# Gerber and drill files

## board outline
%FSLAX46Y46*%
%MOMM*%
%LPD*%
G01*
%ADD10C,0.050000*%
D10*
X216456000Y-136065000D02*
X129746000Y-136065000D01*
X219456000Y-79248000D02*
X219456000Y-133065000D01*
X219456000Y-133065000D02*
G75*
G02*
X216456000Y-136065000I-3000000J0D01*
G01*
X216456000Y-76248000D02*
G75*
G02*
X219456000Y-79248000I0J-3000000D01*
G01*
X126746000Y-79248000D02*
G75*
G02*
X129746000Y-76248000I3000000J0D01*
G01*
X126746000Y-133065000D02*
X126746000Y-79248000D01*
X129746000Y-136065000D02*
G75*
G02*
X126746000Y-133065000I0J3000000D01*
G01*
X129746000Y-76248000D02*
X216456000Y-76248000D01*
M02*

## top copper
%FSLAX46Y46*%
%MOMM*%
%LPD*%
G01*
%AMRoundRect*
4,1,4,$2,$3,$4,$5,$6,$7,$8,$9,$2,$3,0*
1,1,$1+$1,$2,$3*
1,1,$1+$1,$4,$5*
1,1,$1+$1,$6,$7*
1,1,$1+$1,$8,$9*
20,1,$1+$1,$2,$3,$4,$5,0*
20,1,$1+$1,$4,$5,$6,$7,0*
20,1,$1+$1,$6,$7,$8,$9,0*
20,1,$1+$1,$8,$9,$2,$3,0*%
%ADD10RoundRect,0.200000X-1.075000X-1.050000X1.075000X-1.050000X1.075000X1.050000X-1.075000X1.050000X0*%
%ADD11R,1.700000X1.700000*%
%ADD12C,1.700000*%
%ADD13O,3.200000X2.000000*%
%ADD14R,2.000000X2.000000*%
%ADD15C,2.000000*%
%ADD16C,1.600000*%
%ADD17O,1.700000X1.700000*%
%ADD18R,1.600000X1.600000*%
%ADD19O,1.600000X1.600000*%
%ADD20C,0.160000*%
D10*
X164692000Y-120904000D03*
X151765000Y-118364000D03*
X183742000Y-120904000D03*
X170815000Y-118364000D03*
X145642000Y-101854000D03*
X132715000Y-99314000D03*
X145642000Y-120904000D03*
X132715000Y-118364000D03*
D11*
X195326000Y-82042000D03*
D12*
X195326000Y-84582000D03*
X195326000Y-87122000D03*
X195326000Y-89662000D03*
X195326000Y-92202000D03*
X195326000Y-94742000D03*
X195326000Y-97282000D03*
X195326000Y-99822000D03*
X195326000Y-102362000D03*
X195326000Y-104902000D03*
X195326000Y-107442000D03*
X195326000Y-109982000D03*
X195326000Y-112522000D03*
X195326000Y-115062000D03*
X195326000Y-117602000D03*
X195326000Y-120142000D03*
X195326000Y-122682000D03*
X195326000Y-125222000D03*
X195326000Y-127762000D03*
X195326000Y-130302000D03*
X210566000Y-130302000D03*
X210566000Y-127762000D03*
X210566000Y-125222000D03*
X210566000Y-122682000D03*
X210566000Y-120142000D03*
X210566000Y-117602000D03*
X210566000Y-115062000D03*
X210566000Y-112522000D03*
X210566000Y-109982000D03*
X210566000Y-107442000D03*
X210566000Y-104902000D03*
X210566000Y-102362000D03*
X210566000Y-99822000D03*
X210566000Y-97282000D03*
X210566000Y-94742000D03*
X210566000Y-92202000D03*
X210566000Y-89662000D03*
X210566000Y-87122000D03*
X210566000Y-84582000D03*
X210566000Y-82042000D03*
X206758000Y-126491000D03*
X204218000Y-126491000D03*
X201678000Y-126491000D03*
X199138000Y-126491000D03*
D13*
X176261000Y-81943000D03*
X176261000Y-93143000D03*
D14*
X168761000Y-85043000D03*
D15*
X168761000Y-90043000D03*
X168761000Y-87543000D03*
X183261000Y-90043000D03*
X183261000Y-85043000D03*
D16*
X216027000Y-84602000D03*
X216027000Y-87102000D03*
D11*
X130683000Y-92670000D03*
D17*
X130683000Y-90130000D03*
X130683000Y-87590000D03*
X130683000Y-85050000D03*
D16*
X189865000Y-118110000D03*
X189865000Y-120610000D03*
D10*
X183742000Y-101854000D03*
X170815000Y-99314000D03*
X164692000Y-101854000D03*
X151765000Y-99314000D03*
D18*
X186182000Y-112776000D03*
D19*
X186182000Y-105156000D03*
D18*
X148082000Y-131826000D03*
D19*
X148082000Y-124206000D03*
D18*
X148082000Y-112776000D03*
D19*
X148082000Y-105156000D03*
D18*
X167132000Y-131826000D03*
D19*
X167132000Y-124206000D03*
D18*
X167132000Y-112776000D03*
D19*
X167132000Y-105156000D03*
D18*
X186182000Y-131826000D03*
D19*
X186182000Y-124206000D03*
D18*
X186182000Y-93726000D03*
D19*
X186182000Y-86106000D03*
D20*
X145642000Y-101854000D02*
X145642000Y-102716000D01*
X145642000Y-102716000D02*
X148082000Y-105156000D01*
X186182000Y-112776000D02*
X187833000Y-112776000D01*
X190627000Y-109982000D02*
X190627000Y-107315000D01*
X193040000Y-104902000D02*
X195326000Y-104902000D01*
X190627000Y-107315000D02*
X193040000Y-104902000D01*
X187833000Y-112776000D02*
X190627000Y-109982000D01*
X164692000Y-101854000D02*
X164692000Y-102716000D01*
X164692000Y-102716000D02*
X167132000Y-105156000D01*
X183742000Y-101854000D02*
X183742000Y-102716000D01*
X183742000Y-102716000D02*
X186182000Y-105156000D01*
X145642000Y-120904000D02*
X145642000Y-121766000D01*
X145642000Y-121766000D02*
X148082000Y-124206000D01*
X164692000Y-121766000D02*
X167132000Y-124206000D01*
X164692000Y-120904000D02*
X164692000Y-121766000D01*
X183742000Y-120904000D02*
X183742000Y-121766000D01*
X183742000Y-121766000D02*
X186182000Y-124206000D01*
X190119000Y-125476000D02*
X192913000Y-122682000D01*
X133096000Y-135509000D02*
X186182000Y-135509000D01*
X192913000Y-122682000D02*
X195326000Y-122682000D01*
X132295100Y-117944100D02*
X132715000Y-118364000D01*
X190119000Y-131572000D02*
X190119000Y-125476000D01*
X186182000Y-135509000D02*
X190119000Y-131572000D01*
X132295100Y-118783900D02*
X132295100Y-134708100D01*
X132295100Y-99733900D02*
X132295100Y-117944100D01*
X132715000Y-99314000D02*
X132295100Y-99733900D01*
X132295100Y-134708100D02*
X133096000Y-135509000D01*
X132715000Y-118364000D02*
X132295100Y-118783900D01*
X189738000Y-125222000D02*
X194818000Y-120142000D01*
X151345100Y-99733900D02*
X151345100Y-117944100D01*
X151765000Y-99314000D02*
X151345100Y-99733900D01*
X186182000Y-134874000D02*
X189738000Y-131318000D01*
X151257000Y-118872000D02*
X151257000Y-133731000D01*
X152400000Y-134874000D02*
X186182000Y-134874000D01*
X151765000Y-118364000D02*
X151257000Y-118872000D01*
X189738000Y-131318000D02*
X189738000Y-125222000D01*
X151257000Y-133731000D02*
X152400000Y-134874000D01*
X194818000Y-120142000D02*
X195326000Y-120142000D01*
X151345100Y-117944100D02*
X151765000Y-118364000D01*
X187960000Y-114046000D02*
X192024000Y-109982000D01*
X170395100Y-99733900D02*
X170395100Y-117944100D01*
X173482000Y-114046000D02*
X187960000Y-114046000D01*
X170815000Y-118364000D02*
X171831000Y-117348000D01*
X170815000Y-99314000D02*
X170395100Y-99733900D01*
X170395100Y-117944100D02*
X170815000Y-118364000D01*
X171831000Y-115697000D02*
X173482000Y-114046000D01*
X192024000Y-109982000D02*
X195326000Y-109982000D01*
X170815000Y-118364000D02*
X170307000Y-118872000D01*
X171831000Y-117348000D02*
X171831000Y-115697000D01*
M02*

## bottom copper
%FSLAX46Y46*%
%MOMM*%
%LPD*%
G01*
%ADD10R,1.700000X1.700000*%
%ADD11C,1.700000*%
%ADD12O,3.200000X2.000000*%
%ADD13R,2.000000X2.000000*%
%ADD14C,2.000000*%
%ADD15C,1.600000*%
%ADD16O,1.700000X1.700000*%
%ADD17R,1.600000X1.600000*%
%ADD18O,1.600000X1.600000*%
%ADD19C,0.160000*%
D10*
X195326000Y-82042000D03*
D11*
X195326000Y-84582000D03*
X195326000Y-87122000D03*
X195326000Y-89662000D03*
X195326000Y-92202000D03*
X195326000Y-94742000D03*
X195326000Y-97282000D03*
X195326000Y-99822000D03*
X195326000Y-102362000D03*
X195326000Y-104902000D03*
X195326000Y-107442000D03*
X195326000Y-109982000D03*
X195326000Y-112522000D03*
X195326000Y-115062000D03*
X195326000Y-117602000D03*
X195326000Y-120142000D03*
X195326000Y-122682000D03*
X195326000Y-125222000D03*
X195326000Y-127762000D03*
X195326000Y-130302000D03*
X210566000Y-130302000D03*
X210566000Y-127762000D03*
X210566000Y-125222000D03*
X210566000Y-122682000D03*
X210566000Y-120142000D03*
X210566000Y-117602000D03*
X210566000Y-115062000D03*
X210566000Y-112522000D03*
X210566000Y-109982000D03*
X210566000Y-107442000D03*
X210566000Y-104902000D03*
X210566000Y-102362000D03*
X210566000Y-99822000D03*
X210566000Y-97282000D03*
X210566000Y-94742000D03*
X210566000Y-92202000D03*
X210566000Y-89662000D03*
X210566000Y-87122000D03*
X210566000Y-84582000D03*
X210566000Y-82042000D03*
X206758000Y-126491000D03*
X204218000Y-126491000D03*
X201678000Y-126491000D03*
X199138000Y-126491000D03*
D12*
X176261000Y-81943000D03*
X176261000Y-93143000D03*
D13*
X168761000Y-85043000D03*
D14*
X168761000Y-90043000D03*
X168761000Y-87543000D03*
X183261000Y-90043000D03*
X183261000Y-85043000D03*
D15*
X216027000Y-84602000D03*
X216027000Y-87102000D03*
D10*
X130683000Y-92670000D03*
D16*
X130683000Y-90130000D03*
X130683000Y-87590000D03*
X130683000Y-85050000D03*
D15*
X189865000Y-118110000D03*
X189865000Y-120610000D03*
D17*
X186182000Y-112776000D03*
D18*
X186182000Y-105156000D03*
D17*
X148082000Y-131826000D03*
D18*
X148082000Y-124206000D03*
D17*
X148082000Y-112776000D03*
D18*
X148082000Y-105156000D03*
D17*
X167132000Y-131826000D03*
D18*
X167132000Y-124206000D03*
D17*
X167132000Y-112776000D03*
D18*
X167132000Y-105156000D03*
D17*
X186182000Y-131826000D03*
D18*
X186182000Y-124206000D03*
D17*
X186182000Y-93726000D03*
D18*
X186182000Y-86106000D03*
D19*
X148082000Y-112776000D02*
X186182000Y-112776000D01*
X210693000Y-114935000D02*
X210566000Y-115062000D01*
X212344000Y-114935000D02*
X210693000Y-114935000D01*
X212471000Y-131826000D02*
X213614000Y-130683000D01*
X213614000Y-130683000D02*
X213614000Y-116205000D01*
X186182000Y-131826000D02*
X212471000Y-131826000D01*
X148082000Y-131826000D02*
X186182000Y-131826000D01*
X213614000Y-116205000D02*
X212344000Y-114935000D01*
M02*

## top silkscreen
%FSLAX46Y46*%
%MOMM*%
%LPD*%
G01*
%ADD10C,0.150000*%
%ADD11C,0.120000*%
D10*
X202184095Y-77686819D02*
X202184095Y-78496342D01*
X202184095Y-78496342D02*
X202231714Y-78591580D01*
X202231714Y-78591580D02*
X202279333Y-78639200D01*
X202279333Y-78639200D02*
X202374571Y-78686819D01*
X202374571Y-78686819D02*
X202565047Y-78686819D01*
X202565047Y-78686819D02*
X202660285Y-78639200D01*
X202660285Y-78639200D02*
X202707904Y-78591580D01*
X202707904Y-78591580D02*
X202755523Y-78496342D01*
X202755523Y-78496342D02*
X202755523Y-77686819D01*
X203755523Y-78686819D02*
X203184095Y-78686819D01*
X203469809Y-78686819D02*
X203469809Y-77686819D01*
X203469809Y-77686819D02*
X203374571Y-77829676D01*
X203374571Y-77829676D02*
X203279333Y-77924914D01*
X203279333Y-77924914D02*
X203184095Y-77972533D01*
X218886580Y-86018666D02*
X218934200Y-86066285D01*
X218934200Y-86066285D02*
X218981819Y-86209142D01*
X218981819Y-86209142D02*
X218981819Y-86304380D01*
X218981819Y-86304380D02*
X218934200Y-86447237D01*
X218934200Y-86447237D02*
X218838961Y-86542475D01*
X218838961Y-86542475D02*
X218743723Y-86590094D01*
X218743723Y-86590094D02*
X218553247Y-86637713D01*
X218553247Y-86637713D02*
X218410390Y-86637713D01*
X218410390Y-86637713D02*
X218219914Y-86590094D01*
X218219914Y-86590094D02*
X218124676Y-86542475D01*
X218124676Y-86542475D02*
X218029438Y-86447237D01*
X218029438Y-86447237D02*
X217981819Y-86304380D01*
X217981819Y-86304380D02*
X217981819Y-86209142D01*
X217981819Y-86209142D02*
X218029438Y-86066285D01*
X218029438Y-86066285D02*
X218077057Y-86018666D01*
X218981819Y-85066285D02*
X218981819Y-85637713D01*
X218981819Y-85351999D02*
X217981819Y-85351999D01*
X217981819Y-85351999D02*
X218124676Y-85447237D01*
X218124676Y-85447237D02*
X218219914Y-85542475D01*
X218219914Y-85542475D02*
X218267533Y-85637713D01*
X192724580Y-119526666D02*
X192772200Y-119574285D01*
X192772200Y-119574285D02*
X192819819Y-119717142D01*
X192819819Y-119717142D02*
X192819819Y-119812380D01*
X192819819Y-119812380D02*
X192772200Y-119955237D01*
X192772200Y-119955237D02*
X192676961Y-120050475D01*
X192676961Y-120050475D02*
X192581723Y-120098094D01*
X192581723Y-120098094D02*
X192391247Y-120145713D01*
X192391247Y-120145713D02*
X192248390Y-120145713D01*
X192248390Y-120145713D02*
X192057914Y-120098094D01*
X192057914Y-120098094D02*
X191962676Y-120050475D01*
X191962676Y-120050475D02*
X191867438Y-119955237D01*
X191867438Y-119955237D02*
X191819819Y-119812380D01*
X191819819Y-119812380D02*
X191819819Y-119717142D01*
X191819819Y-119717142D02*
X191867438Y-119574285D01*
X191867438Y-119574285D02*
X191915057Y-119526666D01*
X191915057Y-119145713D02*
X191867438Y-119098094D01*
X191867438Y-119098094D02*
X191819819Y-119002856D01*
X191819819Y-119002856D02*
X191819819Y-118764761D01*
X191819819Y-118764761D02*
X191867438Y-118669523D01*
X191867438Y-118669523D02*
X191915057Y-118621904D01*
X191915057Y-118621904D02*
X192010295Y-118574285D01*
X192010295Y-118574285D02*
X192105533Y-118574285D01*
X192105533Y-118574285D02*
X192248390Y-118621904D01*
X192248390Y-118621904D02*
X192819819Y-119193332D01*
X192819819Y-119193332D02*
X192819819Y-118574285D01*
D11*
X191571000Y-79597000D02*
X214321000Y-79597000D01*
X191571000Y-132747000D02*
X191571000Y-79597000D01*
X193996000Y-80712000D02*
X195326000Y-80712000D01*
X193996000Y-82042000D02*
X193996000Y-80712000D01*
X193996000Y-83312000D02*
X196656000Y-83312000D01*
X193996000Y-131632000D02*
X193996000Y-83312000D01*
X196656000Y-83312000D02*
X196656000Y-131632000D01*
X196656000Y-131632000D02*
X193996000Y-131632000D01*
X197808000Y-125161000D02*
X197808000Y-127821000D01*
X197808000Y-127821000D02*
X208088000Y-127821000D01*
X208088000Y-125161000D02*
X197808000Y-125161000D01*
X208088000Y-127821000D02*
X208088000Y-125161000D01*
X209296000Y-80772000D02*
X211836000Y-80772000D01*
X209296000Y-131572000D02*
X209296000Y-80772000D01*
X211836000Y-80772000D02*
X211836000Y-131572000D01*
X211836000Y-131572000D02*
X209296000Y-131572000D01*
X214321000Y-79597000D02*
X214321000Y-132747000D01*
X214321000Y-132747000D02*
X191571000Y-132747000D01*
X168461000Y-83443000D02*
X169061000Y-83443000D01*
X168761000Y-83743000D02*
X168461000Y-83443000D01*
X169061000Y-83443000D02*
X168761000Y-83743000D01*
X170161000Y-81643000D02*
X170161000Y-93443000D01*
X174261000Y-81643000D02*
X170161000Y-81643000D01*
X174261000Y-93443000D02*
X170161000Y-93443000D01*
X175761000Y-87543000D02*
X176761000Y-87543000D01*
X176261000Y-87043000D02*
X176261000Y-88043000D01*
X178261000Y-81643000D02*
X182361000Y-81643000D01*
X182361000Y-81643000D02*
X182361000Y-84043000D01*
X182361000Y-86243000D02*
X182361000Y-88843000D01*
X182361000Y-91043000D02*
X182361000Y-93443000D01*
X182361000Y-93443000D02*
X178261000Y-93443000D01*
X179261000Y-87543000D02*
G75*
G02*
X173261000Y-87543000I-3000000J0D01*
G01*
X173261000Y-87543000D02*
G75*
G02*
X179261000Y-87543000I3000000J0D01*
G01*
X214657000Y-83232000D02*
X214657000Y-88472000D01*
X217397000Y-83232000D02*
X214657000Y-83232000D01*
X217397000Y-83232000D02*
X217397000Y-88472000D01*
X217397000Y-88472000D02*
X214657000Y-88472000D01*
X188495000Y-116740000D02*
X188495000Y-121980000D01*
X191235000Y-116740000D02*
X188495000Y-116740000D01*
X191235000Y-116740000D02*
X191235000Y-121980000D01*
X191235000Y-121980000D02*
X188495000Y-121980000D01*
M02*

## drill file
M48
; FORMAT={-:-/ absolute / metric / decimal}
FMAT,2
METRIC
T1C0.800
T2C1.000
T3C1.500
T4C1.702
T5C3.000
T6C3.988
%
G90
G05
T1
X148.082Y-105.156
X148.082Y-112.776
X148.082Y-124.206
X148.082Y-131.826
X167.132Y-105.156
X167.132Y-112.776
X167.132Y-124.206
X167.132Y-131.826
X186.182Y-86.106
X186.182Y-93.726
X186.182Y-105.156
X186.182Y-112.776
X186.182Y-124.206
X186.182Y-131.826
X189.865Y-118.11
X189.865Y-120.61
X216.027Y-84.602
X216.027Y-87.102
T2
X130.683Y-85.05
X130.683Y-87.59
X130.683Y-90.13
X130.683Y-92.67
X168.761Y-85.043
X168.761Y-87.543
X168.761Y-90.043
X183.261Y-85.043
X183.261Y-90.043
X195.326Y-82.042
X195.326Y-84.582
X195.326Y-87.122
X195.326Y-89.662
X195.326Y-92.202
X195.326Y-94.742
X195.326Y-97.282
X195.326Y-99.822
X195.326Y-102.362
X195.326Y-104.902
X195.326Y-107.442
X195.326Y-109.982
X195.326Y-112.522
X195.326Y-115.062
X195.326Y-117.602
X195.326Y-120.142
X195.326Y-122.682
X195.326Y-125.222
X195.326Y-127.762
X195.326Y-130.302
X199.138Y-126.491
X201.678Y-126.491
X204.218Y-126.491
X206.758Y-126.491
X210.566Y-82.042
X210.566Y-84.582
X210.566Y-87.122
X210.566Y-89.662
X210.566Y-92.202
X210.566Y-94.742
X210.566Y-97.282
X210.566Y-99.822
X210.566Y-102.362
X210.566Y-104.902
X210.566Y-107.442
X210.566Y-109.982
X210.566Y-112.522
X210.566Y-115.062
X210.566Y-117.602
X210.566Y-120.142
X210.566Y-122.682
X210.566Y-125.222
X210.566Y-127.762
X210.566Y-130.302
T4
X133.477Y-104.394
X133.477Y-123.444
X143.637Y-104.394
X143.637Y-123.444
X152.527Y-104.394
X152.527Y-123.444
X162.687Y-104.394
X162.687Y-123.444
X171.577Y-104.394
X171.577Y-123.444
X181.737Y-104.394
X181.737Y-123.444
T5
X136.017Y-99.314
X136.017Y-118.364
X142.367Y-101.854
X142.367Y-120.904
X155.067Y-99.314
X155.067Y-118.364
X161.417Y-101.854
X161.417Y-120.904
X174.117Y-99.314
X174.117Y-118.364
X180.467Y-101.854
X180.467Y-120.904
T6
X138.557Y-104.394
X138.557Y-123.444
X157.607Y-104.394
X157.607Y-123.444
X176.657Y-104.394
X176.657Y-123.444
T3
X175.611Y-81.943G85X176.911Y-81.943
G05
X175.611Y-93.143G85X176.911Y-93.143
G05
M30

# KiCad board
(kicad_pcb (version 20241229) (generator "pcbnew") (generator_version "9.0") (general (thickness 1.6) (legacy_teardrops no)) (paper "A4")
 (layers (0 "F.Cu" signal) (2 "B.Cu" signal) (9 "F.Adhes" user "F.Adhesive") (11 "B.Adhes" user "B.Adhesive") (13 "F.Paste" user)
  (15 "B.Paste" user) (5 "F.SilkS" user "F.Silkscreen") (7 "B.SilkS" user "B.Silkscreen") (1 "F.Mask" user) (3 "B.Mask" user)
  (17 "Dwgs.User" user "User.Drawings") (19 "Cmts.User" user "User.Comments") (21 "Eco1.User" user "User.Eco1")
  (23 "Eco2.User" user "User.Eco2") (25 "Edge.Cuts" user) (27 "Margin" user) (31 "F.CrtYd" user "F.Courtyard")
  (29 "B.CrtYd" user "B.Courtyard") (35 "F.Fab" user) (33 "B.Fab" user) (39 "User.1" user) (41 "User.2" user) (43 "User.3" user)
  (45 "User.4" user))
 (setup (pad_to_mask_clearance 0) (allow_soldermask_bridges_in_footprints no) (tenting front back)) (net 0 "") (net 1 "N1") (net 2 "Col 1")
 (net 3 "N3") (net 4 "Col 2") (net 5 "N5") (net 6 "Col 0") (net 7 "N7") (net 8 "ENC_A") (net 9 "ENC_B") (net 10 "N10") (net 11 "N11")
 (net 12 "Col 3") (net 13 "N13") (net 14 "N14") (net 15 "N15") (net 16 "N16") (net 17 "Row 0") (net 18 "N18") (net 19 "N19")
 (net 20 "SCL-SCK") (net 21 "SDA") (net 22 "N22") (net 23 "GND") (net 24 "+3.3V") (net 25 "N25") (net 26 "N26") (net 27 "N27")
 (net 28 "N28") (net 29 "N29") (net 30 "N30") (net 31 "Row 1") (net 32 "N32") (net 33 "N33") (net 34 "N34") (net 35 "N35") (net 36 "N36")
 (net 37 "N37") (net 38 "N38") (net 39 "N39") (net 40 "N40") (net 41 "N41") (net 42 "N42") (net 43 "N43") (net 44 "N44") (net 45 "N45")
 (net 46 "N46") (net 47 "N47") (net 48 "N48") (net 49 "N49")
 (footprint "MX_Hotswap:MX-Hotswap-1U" (layer "F.Cu") (at 157.607 123.444)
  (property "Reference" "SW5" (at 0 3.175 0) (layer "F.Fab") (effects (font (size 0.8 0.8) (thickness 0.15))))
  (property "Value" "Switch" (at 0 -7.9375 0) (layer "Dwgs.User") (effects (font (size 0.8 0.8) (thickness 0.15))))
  (pad "" np_thru_hole circle (at -5.08 0 311.901) (size 1.7018 1.7018) (drill 1.7018) (layers "*.Cu" "*.Mask"))
  (pad "" np_thru_hole circle (at -2.54 -5.08) (size 3 3) (drill 3) (layers "*.Cu" "*.Mask"))
  (pad "" np_thru_hole circle (at 0 0) (size 3.9878 3.9878) (drill 3.9878) (layers "*.Cu" "*.Mask"))
  (pad "" np_thru_hole circle (at 3.81 -2.54) (size 3 3) (drill 3) (layers "*.Cu" "*.Mask"))
  (pad "" np_thru_hole circle (at 5.08 0 311.901) (size 1.7018 1.7018) (drill 1.7018) (layers "*.Cu" "*.Mask"))
  (pad "1" smd roundrect (at 7.085 -2.54) (size 2.55 2.5) (layers "F.Cu" "F.Mask" "F.Paste") (roundrect_rratio 0.08) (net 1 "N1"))
  (pad "2" smd roundrect (at -5.842 -5.08) (size 2.55 2.5) (layers "F.Cu" "F.Mask" "F.Paste") (roundrect_rratio 0.08) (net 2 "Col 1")))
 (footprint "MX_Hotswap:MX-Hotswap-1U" (layer "F.Cu") (at 176.657 123.444)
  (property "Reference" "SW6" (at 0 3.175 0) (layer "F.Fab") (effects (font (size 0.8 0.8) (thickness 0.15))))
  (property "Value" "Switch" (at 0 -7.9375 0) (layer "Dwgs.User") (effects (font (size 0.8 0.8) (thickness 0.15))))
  (pad "" np_thru_hole circle (at -5.08 0 311.901) (size 1.7018 1.7018) (drill 1.7018) (layers "*.Cu" "*.Mask"))
  (pad "" np_thru_hole circle (at -2.54 -5.08) (size 3 3) (drill 3) (layers "*.Cu" "*.Mask"))
  (pad "" np_thru_hole circle (at 0 0) (size 3.9878 3.9878) (drill 3.9878) (layers "*.Cu" "*.Mask"))
  (pad "" np_thru_hole circle (at 3.81 -2.54) (size 3 3) (drill 3) (layers "*.Cu" "*.Mask"))
  (pad "" np_thru_hole circle (at 5.08 0 311.901) (size 1.7018 1.7018) (drill 1.7018) (layers "*.Cu" "*.Mask"))
  (pad "1" smd roundrect (at 7.085 -2.54) (size 2.55 2.5) (layers "F.Cu" "F.Mask" "F.Paste") (roundrect_rratio 0.08) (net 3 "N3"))
  (pad "2" smd roundrect (at -5.842 -5.08) (size 2.55 2.5) (layers "F.Cu" "F.Mask" "F.Paste") (roundrect_rratio 0.08) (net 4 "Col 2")))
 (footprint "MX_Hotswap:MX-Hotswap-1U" (layer "F.Cu") (at 138.557 104.394)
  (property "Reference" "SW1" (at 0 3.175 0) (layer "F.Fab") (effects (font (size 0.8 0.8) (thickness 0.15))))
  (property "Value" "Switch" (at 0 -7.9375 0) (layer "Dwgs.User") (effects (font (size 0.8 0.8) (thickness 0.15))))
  (pad "" np_thru_hole circle (at -5.08 0 311.901) (size 1.7018 1.7018) (drill 1.7018) (layers "*.Cu" "*.Mask"))
  (pad "" np_thru_hole circle (at -2.54 -5.08) (size 3 3) (drill 3) (layers "*.Cu" "*.Mask"))
  (pad "" np_thru_hole circle (at 0 0) (size 3.9878 3.9878) (drill 3.9878) (layers "*.Cu" "*.Mask"))
  (pad "" np_thru_hole circle (at 3.81 -2.54) (size 3 3) (drill 3) (layers "*.Cu" "*.Mask"))
  (pad "" np_thru_hole circle (at 5.08 0 311.901) (size 1.7018 1.7018) (drill 1.7018) (layers "*.Cu" "*.Mask"))
  (pad "1" smd roundrect (at 7.085 -2.54) (size 2.55 2.5) (layers "F.Cu" "F.Mask" "F.Paste") (roundrect_rratio 0.08) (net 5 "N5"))
  (pad "2" smd roundrect (at -5.842 -5.08) (size 2.55 2.5) (layers "F.Cu" "F.Mask" "F.Paste") (roundrect_rratio 0.08) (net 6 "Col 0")))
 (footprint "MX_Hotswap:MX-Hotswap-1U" (layer "F.Cu") (at 138.557 123.444)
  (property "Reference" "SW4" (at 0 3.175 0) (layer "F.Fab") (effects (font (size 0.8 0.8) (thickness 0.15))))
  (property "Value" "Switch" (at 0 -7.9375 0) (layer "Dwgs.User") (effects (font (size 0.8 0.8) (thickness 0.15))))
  (pad "" np_thru_hole circle (at -5.08 0 311.901) (size 1.7018 1.7018) (drill 1.7018) (layers "*.Cu" "*.Mask"))
  (pad "" np_thru_hole circle (at -2.54 -5.08) (size 3 3) (drill 3) (layers "*.Cu" "*.Mask"))
  (pad "" np_thru_hole circle (at 0 0) (size 3.9878 3.9878) (drill 3.9878) (layers "*.Cu" "*.Mask"))
  (pad "" np_thru_hole circle (at 3.81 -2.54) (size 3 3) (drill 3) (layers "*.Cu" "*.Mask"))
  (pad "" np_thru_hole circle (at 5.08 0 311.901) (size 1.7018 1.7018) (drill 1.7018) (layers "*.Cu" "*.Mask"))
  (pad "1" smd roundrect (at 7.085 -2.54) (size 2.55 2.5) (layers "F.Cu" "F.Mask" "F.Paste") (roundrect_rratio 0.08) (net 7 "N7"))
  (pad "2" smd roundrect (at -5.842 -5.08) (size 2.55 2.5) (layers "F.Cu" "F.Mask" "F.Paste") (roundrect_rratio 0.08) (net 6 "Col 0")))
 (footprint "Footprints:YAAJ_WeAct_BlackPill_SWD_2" (layer "F.Cu") (at 195.326 82.042)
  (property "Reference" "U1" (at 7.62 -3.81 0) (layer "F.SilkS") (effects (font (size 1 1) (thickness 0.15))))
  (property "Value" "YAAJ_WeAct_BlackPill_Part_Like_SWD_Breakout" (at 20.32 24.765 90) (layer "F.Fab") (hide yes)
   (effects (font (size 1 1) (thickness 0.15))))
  (fp_line (start -3.755 -2.445) (end 18.995 -2.445) (stroke (width 0.12) (type solid)) (layer "F.SilkS"))
  (fp_line (start -3.755 50.705) (end -3.755 -2.445) (stroke (width 0.12) (type solid)) (layer "F.SilkS"))
  (fp_line (start -1.33 -1.33) (end 0 -1.33) (stroke (width 0.12) (type solid)) (layer "F.SilkS"))
  (fp_line (start -1.33 0) (end -1.33 -1.33) (stroke (width 0.12) (type solid)) (layer "F.SilkS"))
  (fp_line (start -1.33 1.27) (end 1.33 1.27) (stroke (width 0.12) (type solid)) (layer "F.SilkS"))
  (fp_line (start -1.33 49.59) (end -1.33 1.27) (stroke (width 0.12) (type solid)) (layer "F.SilkS"))
  (fp_line (start 1.33 1.27) (end 1.33 49.59) (stroke (width 0.12) (type solid)) (layer "F.SilkS"))
  (fp_line (start 1.33 49.59) (end -1.33 49.59) (stroke (width 0.12) (type solid)) (layer "F.SilkS"))
  (fp_line (start 2.482 43.119) (end 2.482 45.779) (stroke (width 0.12) (type solid)) (layer "F.SilkS"))
  (fp_line (start 2.482 45.779) (end 12.762 45.779) (stroke (width 0.12) (type solid)) (layer "F.SilkS"))
  (fp_line (start 12.762 43.119) (end 2.482 43.119) (stroke (width 0.12) (type solid)) (layer "F.SilkS"))
  (fp_line (start 12.762 45.779) (end 12.762 43.119) (stroke (width 0.12) (type solid)) (layer "F.SilkS"))
  (fp_line (start 13.97 -1.27) (end 16.51 -1.27) (stroke (width 0.12) (type solid)) (layer "F.SilkS"))
  (fp_line (start 13.97 49.53) (end 13.97 -1.27) (stroke (width 0.12) (type solid)) (layer "F.SilkS"))
  (fp_line (start 16.51 -1.27) (end 16.51 49.53) (stroke (width 0.12) (type solid)) (layer "F.SilkS"))
  (fp_line (start 16.51 49.53) (end 13.97 49.53) (stroke (width 0.12) (type solid)) (layer "F.SilkS"))
  (fp_line (start 18.995 -2.445) (end 18.995 50.705) (stroke (width 0.12) (type solid)) (layer "F.SilkS"))
  (fp_line (start 18.995 50.705) (end -3.755 50.705) (stroke (width 0.12) (type solid)) (layer "F.SilkS"))
  (pad "1" thru_hole rect (at 0 0) (size 1.7 1.7) (drill 1) (layers "*.Cu" "*.Mask") (remove_unused_layers no) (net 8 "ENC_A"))
  (pad "2" thru_hole circle (at 0 2.54) (size 1.7 1.7) (drill 1) (layers "*.Cu" "*.Mask") (remove_unused_layers no) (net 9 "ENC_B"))
  (pad "3" thru_hole circle (at 0 5.08) (size 1.7 1.7) (drill 1) (layers "*.Cu" "*.Mask") (remove_unused_layers no) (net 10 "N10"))
  (pad "4" thru_hole circle (at 0 7.62) (size 1.7 1.7) (drill 1) (layers "*.Cu" "*.Mask") (remove_unused_layers no) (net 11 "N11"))
  (pad "5" thru_hole circle (at 0 10.16) (size 1.7 1.7) (drill 1) (layers "*.Cu" "*.Mask") (remove_unused_layers no) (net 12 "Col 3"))
  (pad "6" thru_hole circle (at 0 12.7) (size 1.7 1.7) (drill 1) (layers "*.Cu" "*.Mask") (remove_unused_layers no) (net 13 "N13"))
  (pad "7" thru_hole circle (at 0 15.24) (size 1.7 1.7) (drill 1) (layers "*.Cu" "*.Mask") (remove_unused_layers no) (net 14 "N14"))
  (pad "8" thru_hole circle (at 0 17.78) (size 1.7 1.7) (drill 1) (layers "*.Cu" "*.Mask") (remove_unused_layers no) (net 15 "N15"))
  (pad "9" thru_hole circle (at 0 20.32) (size 1.7 1.7) (drill 1) (layers "*.Cu" "*.Mask") (remove_unused_layers no) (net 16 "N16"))
  (pad "10" thru_hole circle (at 0 22.86) (size 1.7 1.7) (drill 1) (layers "*.Cu" "*.Mask") (remove_unused_layers no) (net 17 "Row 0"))
  (pad "11" thru_hole circle (at 0 25.4) (size 1.7 1.7) (drill 1) (layers "*.Cu" "*.Mask") (remove_unused_layers no) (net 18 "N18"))
  (pad "12" thru_hole circle (at 0 27.94) (size 1.7 1.7) (drill 1) (layers "*.Cu" "*.Mask") (remove_unused_layers no) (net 4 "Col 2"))
  (pad "13" thru_hole circle (at 0 30.48) (size 1.7 1.7) (drill 1) (layers "*.Cu" "*.Mask") (remove_unused_layers no) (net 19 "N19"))
  (pad "14" thru_hole circle (at 0 33.02) (size 1.7 1.7) (drill 1) (layers "*.Cu" "*.Mask") (remove_unused_layers no) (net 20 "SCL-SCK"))
  (pad "15" thru_hole circle (at 0 35.56) (size 1.7 1.7) (drill 1) (layers "*.Cu" "*.Mask") (remove_unused_layers no) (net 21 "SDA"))
  (pad "16" thru_hole circle (at 0 38.1) (size 1.7 1.7) (drill 1) (layers "*.Cu" "*.Mask") (remove_unused_layers no) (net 2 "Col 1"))
  (pad "17" thru_hole circle (at 0 40.64) (size 1.7 1.7) (drill 1) (layers "*.Cu" "*.Mask") (remove_unused_layers no) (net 6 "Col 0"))
  (pad "18" thru_hole circle (at 0 43.18) (size 1.7 1.7) (drill 1) (layers "*.Cu" "*.Mask") (remove_unused_layers no) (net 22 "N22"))
  (pad "19" thru_hole circle (at 0 45.72) (size 1.7 1.7) (drill 1) (layers "*.Cu" "*.Mask") (remove_unused_layers no) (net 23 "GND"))
  (pad "20" thru_hole circle (at 0 48.26) (size 1.7 1.7) (drill 1) (layers "*.Cu" "*.Mask") (remove_unused_layers no) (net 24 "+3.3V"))
  (pad "21" thru_hole circle (at 15.24 48.26) (size 1.7 1.7) (drill 1) (layers "*.Cu" "*.Mask") (remove_unused_layers no) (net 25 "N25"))
  (pad "22" thru_hole circle (at 15.24 45.72) (size 1.7 1.7) (drill 1) (layers "*.Cu" "*.Mask") (remove_unused_layers no) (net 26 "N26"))
  (pad "23" thru_hole circle (at 15.24 43.18) (size 1.7 1.7) (drill 1) (layers "*.Cu" "*.Mask") (remove_unused_layers no) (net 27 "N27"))
  (pad "24" thru_hole circle (at 15.24 40.64) (size 1.7 1.7) (drill 1) (layers "*.Cu" "*.Mask") (remove_unused_layers no) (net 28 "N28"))
  (pad "25" thru_hole circle (at 15.24 38.1) (size 1.7 1.7) (drill 1) (layers "*.Cu" "*.Mask") (remove_unused_layers no) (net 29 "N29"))
  (pad "26" thru_hole circle (at 15.24 35.56) (size 1.7 1.7) (drill 1) (layers "*.Cu" "*.Mask") (remove_unused_layers no) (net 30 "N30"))
  (pad "27" thru_hole circle (at 15.24 33.02) (size 1.7 1.7) (drill 1) (layers "*.Cu" "*.Mask") (remove_unused_layers no) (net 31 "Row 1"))
  (pad "28" thru_hole circle (at 15.24 30.48) (size 1.7 1.7) (drill 1) (layers "*.Cu" "*.Mask") (remove_unused_layers no) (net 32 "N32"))
  (pad "29" thru_hole circle (at 15.24 27.94) (size 1.7 1.7) (drill 1) (layers "*.Cu" "*.Mask") (remove_unused_layers no) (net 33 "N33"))
  (pad "30" thru_hole circle (at 15.24 25.4) (size 1.7 1.7) (drill 1) (layers "*.Cu" "*.Mask") (remove_unused_layers no) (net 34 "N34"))
  (pad "31" thru_hole circle (at 15.24 22.86) (size 1.7 1.7) (drill 1) (layers "*.Cu" "*.Mask") (remove_unused_layers no) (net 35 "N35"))
  (pad "32" thru_hole circle (at 15.24 20.32) (size 1.7 1.7) (drill 1) (layers "*.Cu" "*.Mask") (remove_unused_layers no) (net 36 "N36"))
  (pad "33" thru_hole circle (at 15.24 17.78) (size 1.7 1.7) (drill 1) (layers "*.Cu" "*.Mask") (remove_unused_layers no) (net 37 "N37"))
  (pad "34" thru_hole circle (at 15.24 15.24) (size 1.7 1.7) (drill 1) (layers "*.Cu" "*.Mask") (remove_unused_layers no) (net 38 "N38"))
  (pad "35" thru_hole circle (at 15.24 12.7) (size 1.7 1.7) (drill 1) (layers "*.Cu" "*.Mask") (remove_unused_layers no) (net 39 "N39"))
  (pad "36" thru_hole circle (at 15.24 10.16) (size 1.7 1.7) (drill 1) (layers "*.Cu" "*.Mask") (remove_unused_layers no) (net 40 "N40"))
  (pad "37" thru_hole circle (at 15.24 7.62) (size 1.7 1.7) (drill 1) (layers "*.Cu" "*.Mask") (remove_unused_layers no) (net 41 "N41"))
  (pad "38" thru_hole circle (at 15.24 5.08) (size 1.7 1.7) (drill 1) (layers "*.Cu" "*.Mask") (remove_unused_layers no) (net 24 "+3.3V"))
  (pad "39" thru_hole circle (at 15.24 2.54) (size 1.7 1.7) (drill 1) (layers "*.Cu" "*.Mask") (remove_unused_layers no) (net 23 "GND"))
  (pad "40" thru_hole circle (at 15.24 0) (size 1.7 1.7) (drill 1) (layers "*.Cu" "*.Mask") (remove_unused_layers no) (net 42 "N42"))
  (pad "41" thru_hole circle (at 11.432 44.449) (size 1.7 1.7) (drill 1) (layers "*.Cu" "*.Mask") (remove_unused_layers no) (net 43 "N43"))
  (pad "42" thru_hole circle (at 8.892 44.449) (size 1.7 1.7) (drill 1) (layers "*.Cu" "*.Mask") (remove_unused_layers no) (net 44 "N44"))
  (pad "43" thru_hole circle (at 6.352 44.449) (size 1.7 1.7) (drill 1) (layers "*.Cu" "*.Mask") (remove_unused_layers no) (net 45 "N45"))
  (pad "44" thru_hole circle (at 3.812 44.449) (size 1.7 1.7) (drill 1) (layers "*.Cu" "*.Mask") (remove_unused_layers no) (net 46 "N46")))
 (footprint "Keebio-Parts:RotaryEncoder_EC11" (layer "F.Cu") (at 176.261 87.543)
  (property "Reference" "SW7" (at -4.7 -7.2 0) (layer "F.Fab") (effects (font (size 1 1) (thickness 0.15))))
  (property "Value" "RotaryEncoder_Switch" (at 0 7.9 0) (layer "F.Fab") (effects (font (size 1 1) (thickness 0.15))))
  (fp_line (start -7.8 -4.1) (end -7.2 -4.1) (stroke (width 0.12) (type solid)) (layer "F.SilkS"))
  (fp_line (start -7.5 -3.8) (end -7.8 -4.1) (stroke (width 0.12) (type solid)) (layer "F.SilkS"))
  (fp_line (start -7.2 -4.1) (end -7.5 -3.8) (stroke (width 0.12) (type solid)) (layer "F.SilkS"))
  (fp_line (start -6.1 -5.9) (end -6.1 5.9) (stroke (width 0.12) (type solid)) (layer "F.SilkS"))
  (fp_line (start -2 -5.9) (end -6.1 -5.9) (stroke (width 0.12) (type solid)) (layer "F.SilkS"))
  (fp_line (start -2 5.9) (end -6.1 5.9) (stroke (width 0.12) (type solid)) (layer "F.SilkS"))
  (fp_line (start -0.5 0) (end 0.5 0) (stroke (width 0.12) (type solid)) (layer "F.SilkS"))
  (fp_line (start 0 -0.5) (end 0 0.5) (stroke (width 0.12) (type solid)) (layer "F.SilkS"))
  (fp_line (start 2 -5.9) (end 6.1 -5.9) (stroke (width 0.12) (type solid)) (layer "F.SilkS"))
  (fp_line (start 6.1 -5.9) (end 6.1 -3.5) (stroke (width 0.12) (type solid)) (layer "F.SilkS"))
  (fp_line (start 6.1 -1.3) (end 6.1 1.3) (stroke (width 0.12) (type solid)) (layer "F.SilkS"))
  (fp_line (start 6.1 3.5) (end 6.1 5.9) (stroke (width 0.12) (type solid)) (layer "F.SilkS"))
  (fp_line (start 6.1 5.9) (end 2 5.9) (stroke (width 0.12) (type solid)) (layer "F.SilkS"))
  (fp_circle (center 0 0) (end 3 0) (stroke (width 0.12) (type solid)) (fill no) (layer "F.SilkS"))
  (pad "" np_thru_hole oval (at 0 -5.6) (size 3.2 2) (drill oval 2.8 1.5) (layers "*.Cu" "*.Mask"))
  (pad "" np_thru_hole oval (at 0 5.6) (size 3.2 2) (drill oval 2.8 1.5) (layers "*.Cu" "*.Mask"))
  (pad "A" thru_hole rect (at -7.5 -2.5) (size 2 2) (drill 1) (layers "*.Cu" "*.Mask") (remove_unused_layers no) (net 8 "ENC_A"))
  (pad "B" thru_hole circle (at -7.5 2.5) (size 2 2) (drill 1) (layers "*.Cu" "*.Mask") (remove_unused_layers no) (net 9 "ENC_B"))
  (pad "C" thru_hole circle (at -7.5 0) (size 2 2) (drill 1) (layers "*.Cu" "*.Mask") (remove_unused_layers no) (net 23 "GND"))
  (pad "S1" thru_hole circle (at 7 2.5) (size 2 2) (drill 1) (layers "*.Cu" "*.Mask") (remove_unused_layers no) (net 12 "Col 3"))
  (pad "S2" thru_hole circle (at 7 -2.5) (size 2 2) (drill 1) (layers "*.Cu" "*.Mask") (remove_unused_layers no) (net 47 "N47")))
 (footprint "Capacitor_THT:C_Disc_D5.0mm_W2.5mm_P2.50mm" (layer "F.Cu") (at 216.027 84.602 -90)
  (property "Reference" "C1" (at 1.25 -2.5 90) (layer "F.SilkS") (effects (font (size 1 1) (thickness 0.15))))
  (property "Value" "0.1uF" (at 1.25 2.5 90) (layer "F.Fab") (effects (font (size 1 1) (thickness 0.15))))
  (fp_line (start -1.37 1.37) (end 3.87 1.37) (stroke (width 0.12) (type solid)) (layer "F.SilkS"))
  (fp_line (start -1.37 -1.37) (end -1.37 1.37) (stroke (width 0.12) (type solid)) (layer "F.SilkS"))
  (fp_line (start -1.37 -1.37) (end 3.87 -1.37) (stroke (width 0.12) (type solid)) (layer "F.SilkS"))
  (fp_line (start 3.87 -1.37) (end 3.87 1.37) (stroke (width 0.12) (type solid)) (layer "F.SilkS"))
  (pad "1" thru_hole circle (at 0 0 270) (size 1.6 1.6) (drill 0.8) (layers "*.Cu" "*.Mask") (remove_unused_layers no) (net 23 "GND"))
  (pad "2" thru_hole circle (at 2.5 0 270) (size 1.6 1.6) (drill 0.8) (layers "*.Cu" "*.Mask") (remove_unused_layers no) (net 24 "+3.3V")))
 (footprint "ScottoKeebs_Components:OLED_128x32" (layer "F.Cu") (at 129.083 82.87)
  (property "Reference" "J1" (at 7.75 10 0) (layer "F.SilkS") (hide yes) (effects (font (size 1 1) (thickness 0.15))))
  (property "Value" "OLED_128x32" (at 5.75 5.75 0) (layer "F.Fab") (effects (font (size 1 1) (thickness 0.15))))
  (pad "1" thru_hole rect (at 1.6 9.8 180) (size 1.7 1.7) (drill 1) (layers "*.Cu" "*.Mask") (remove_unused_layers no) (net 23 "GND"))
  (pad "2" thru_hole oval (at 1.6 7.26 180) (size 1.7 1.7) (drill 1) (layers "*.Cu" "*.Mask") (remove_unused_layers no) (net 24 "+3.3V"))
  (pad "3" thru_hole oval (at 1.6 4.72 180) (size 1.7 1.7) (drill 1) (layers "*.Cu" "*.Mask") (remove_unused_layers no) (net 20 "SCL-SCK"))
  (pad "4" thru_hole oval (at 1.6 2.18 180) (size 1.7 1.7) (drill 1) (layers "*.Cu" "*.Mask") (remove_unused_layers no) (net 21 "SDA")))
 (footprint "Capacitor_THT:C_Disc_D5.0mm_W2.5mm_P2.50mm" (layer "F.Cu") (at 189.865 118.11 -90)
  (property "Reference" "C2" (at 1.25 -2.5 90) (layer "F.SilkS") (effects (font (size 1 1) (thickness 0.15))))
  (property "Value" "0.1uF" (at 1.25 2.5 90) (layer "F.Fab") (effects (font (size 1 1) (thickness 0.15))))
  (fp_line (start -1.37 1.37) (end 3.87 1.37) (stroke (width 0.12) (type solid)) (layer "F.SilkS"))
  (fp_line (start -1.37 -1.37) (end -1.37 1.37) (stroke (width 0.12) (type solid)) (layer "F.SilkS"))
  (fp_line (start -1.37 -1.37) (end 3.87 -1.37) (stroke (width 0.12) (type solid)) (layer "F.SilkS"))
  (fp_line (start 3.87 -1.37) (end 3.87 1.37) (stroke (width 0.12) (type solid)) (layer "F.SilkS"))
  (pad "1" thru_hole circle (at 0 0 270) (size 1.6 1.6) (drill 0.8) (layers "*.Cu" "*.Mask") (remove_unused_layers no) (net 23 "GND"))
  (pad "2" thru_hole circle (at 2.5 0 270) (size 1.6 1.6) (drill 0.8) (layers "*.Cu" "*.Mask") (remove_unused_layers no) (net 24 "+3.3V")))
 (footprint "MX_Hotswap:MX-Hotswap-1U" (layer "F.Cu") (at 176.657 104.394)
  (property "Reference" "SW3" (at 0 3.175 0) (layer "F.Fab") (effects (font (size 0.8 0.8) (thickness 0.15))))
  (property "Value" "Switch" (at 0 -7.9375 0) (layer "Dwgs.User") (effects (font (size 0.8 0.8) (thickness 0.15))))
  (pad "" np_thru_hole circle (at -5.08 0 311.901) (size 1.7018 1.7018) (drill 1.7018) (layers "*.Cu" "*.Mask"))
  (pad "" np_thru_hole circle (at -2.54 -5.08) (size 3 3) (drill 3) (layers "*.Cu" "*.Mask"))
  (pad "" np_thru_hole circle (at 0 0) (size 3.9878 3.9878) (drill 3.9878) (layers "*.Cu" "*.Mask"))
  (pad "" np_thru_hole circle (at 3.81 -2.54) (size 3 3) (drill 3) (layers "*.Cu" "*.Mask"))
  (pad "" np_thru_hole circle (at 5.08 0 311.901) (size 1.7018 1.7018) (drill 1.7018) (layers "*.Cu" "*.Mask"))
  (pad "1" smd roundrect (at 7.085 -2.54) (size 2.55 2.5) (layers "F.Cu" "F.Mask" "F.Paste") (roundrect_rratio 0.08) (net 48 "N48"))
  (pad "2" smd roundrect (at -5.842 -5.08) (size 2.55 2.5) (layers "F.Cu" "F.Mask" "F.Paste") (roundrect_rratio 0.08) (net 4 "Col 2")))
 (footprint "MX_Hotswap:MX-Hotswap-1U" (layer "F.Cu") (at 157.607 104.394)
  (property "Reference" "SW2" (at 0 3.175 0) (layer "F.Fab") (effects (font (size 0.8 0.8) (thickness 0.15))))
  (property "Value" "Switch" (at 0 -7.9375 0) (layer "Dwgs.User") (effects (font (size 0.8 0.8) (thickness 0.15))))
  (pad "" np_thru_hole circle (at -5.08 0 311.901) (size 1.7018 1.7018) (drill 1.7018) (layers "*.Cu" "*.Mask"))
  (pad "" np_thru_hole circle (at -2.54 -5.08) (size 3 3) (drill 3) (layers "*.Cu" "*.Mask"))
  (pad "" np_thru_hole circle (at 0 0) (size 3.9878 3.9878) (drill 3.9878) (layers "*.Cu" "*.Mask"))
  (pad "" np_thru_hole circle (at 3.81 -2.54) (size 3 3) (drill 3) (layers "*.Cu" "*.Mask"))
  (pad "" np_thru_hole circle (at 5.08 0 311.901) (size 1.7018 1.7018) (drill 1.7018) (layers "*.Cu" "*.Mask"))
  (pad "1" smd roundrect (at 7.085 -2.54) (size 2.55 2.5) (layers "F.Cu" "F.Mask" "F.Paste") (roundrect_rratio 0.08) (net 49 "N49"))
  (pad "2" smd roundrect (at -5.842 -5.08) (size 2.55 2.5) (layers "F.Cu" "F.Mask" "F.Paste") (roundrect_rratio 0.08) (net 2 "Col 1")))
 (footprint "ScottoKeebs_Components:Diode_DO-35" (layer "B.Cu") (at 186.182 112.776 90)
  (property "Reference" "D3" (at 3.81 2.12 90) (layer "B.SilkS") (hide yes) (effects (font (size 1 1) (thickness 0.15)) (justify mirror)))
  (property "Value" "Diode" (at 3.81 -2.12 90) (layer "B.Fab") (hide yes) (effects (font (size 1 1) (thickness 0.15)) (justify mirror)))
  (pad "1" thru_hole rect (at 0 0 90) (size 1.6 1.6) (drill 0.8) (layers "*.Cu" "*.Mask") (remove_unused_layers no) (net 17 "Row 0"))
  (pad "2" thru_hole oval (at 7.62 0 90) (size 1.6 1.6) (drill 0.8) (layers "*.Cu" "*.Mask") (remove_unused_layers no) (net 48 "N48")))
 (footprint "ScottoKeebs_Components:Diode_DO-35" (layer "B.Cu") (at 148.082 131.826 90)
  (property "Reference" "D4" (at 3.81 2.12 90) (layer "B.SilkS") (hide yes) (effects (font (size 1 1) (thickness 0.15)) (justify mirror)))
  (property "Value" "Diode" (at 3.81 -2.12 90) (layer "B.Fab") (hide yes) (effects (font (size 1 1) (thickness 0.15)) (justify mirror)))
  (pad "1" thru_hole rect (at 0 0 90) (size 1.6 1.6) (drill 0.8) (layers "*.Cu" "*.Mask") (remove_unused_layers no) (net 31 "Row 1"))
  (pad "2" thru_hole oval (at 7.62 0 90) (size 1.6 1.6) (drill 0.8) (layers "*.Cu" "*.Mask") (remove_unused_layers no) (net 7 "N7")))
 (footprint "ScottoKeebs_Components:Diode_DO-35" (layer "B.Cu") (at 148.082 112.776 90)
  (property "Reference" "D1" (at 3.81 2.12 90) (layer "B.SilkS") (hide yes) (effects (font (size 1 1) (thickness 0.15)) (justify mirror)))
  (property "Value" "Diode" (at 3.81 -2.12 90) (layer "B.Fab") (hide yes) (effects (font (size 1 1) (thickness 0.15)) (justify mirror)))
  (pad "1" thru_hole rect (at 0 0 90) (size 1.6 1.6) (drill 0.8) (layers "*.Cu" "*.Mask") (remove_unused_layers no) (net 17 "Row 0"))
  (pad "2" thru_hole oval (at 7.62 0 90) (size 1.6 1.6) (drill 0.8) (layers "*.Cu" "*.Mask") (remove_unused_layers no) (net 5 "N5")))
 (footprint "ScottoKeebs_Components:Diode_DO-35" (layer "B.Cu") (at 167.132 131.826 90)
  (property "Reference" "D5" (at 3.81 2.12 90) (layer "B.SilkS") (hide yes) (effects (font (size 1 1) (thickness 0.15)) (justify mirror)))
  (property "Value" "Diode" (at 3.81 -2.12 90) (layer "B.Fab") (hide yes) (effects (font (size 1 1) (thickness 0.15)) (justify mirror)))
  (pad "1" thru_hole rect (at 0 0 90) (size 1.6 1.6) (drill 0.8) (layers "*.Cu" "*.Mask") (remove_unused_layers no) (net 31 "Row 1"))
  (pad "2" thru_hole oval (at 7.62 0 90) (size 1.6 1.6) (drill 0.8) (layers "*.Cu" "*.Mask") (remove_unused_layers no) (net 1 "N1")))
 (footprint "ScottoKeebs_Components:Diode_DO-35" (layer "B.Cu") (at 167.132 112.776 90)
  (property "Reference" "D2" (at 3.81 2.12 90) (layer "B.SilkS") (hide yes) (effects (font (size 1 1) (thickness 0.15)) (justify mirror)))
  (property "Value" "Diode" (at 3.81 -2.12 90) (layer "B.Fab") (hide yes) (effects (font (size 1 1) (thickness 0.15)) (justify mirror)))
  (pad "1" thru_hole rect (at 0 0 90) (size 1.6 1.6) (drill 0.8) (layers "*.Cu" "*.Mask") (remove_unused_layers no) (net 17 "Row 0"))
  (pad "2" thru_hole oval (at 7.62 0 90) (size 1.6 1.6) (drill 0.8) (layers "*.Cu" "*.Mask") (remove_unused_layers no) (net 49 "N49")))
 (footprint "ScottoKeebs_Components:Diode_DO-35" (layer "B.Cu") (at 186.182 131.826 90)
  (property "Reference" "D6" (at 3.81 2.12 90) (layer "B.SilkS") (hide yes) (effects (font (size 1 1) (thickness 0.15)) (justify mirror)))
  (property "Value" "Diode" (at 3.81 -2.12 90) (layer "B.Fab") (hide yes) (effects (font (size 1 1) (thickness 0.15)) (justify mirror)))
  (pad "1" thru_hole rect (at 0 0 90) (size 1.6 1.6) (drill 0.8) (layers "*.Cu" "*.Mask") (remove_unused_layers no) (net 31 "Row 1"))
  (pad "2" thru_hole oval (at 7.62 0 90) (size 1.6 1.6) (drill 0.8) (layers "*.Cu" "*.Mask") (remove_unused_layers no) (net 3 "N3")))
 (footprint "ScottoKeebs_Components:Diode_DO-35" (layer "B.Cu") (at 186.182 93.726 90)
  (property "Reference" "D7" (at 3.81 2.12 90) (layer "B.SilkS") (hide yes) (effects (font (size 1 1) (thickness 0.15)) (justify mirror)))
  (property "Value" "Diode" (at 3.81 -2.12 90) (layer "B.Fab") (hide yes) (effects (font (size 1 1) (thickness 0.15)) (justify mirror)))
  (pad "1" thru_hole rect (at 0 0 90) (size 1.6 1.6) (drill 0.8) (layers "*.Cu" "*.Mask") (remove_unused_layers no) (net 17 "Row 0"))
  (pad "2" thru_hole oval (at 7.62 0 90) (size 1.6 1.6) (drill 0.8) (layers "*.Cu" "*.Mask") (remove_unused_layers no) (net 47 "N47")))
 (gr_line (start 216.456 136.065) (end 129.746 136.065) (stroke (width 0.05) (type default)) (layer "Edge.Cuts"))
 (gr_line (start 219.456 79.248) (end 219.456 133.065) (stroke (width 0.05) (type default)) (layer "Edge.Cuts"))
 (gr_arc (start 219.456 133.065) (mid 218.57732 135.18632) (end 216.456 136.065) (stroke (width 0.05) (type default)) (layer "Edge.Cuts"))
 (gr_arc (start 216.456 76.248) (mid 218.57732 77.12668) (end 219.456 79.248) (stroke (width 0.05) (type default)) (layer "Edge.Cuts"))
 (gr_arc (start 126.746 79.248) (mid 127.62468 77.12668) (end 129.746 76.248) (stroke (width 0.05) (type default)) (layer "Edge.Cuts"))
 (gr_line (start 126.746 133.065) (end 126.746 79.248) (stroke (width 0.05) (type default)) (layer "Edge.Cuts"))
 (gr_arc (start 129.746 136.065) (mid 127.62468 135.18632) (end 126.746 133.065) (stroke (width 0.05) (type default)) (layer "Edge.Cuts"))
 (gr_line (start 129.746 76.248) (end 216.456 76.248) (stroke (width 0.05) (type default)) (layer "Edge.Cuts"))
 (segment (start 145.642 101.854) (end 145.642 102.716) (width 0.16) (layer "F.Cu") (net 5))
 (segment (start 145.642 102.716) (end 148.082 105.156) (width 0.16) (layer "F.Cu") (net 5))
 (segment (start 186.182 112.776) (end 187.833 112.776) (width 0.16) (layer "F.Cu") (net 17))
 (segment (start 190.627 109.982) (end 190.627 107.315) (width 0.16) (layer "F.Cu") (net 17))
 (segment (start 193.04 104.902) (end 195.326 104.902) (width 0.16) (layer "F.Cu") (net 17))
 (segment (start 190.627 107.315) (end 193.04 104.902) (width 0.16) (layer "F.Cu") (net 17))
 (segment (start 187.833 112.776) (end 190.627 109.982) (width 0.16) (layer "F.Cu") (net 17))
 (segment (start 148.082 112.776) (end 186.182 112.776) (width 0.16) (layer "B.Cu") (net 17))
 (segment (start 164.692 101.854) (end 164.692 102.716) (width 0.16) (layer "F.Cu") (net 49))
 (segment (start 164.692 102.716) (end 167.132 105.156) (width 0.16) (layer "F.Cu") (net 49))
 (segment (start 183.742 101.854) (end 183.742 102.716) (width 0.16) (layer "F.Cu") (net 48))
 (segment (start 183.742 102.716) (end 186.182 105.156) (width 0.16) (layer "F.Cu") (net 48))
 (segment (start 145.642 120.904) (end 145.642 121.766) (width 0.16) (layer "F.Cu") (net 7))
 (segment (start 145.642 121.766) (end 148.082 124.206) (width 0.16) (layer "F.Cu") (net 7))
 (segment (start 210.693 114.935) (end 210.566 115.062) (width 0.16) (layer "B.Cu") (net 31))
 (segment (start 212.344 114.935) (end 210.693 114.935) (width 0.16) (layer "B.Cu") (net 31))
 (segment (start 212.471 131.826) (end 213.614 130.683) (width 0.16) (layer "B.Cu") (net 31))
 (segment (start 213.614 130.683) (end 213.614 116.205) (width 0.16) (layer "B.Cu") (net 31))
 (segment (start 186.182 131.826) (end 212.471 131.826) (width 0.16) (layer "B.Cu") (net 31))
 (segment (start 148.082 131.826) (end 186.182 131.826) (width 0.16) (layer "B.Cu") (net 31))
 (segment (start 213.614 116.205) (end 212.344 114.935) (width 0.16) (layer "B.Cu") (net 31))
 (segment (start 164.692 121.766) (end 167.132 124.206) (width 0.16) (layer "F.Cu") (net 1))
 (segment (start 164.692 120.904) (end 164.692 121.766) (width 0.16) (layer "F.Cu") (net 1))
 (segment (start 183.742 120.904) (end 183.742 121.766) (width 0.16) (layer "F.Cu") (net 3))
 (segment (start 183.742 121.766) (end 186.182 124.206) (width 0.16) (layer "F.Cu") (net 3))
 (segment (start 190.119 125.476) (end 192.913 122.682) (width 0.16) (layer "F.Cu") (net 6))
 (segment (start 133.096 135.509) (end 186.182 135.509) (width 0.16) (layer "F.Cu") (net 6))
 (segment (start 192.913 122.682) (end 195.326 122.682) (width 0.16) (layer "F.Cu") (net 6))
 (segment (start 132.2951 117.9441) (end 132.715 118.364) (width 0.16) (layer "F.Cu") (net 6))
 (segment (start 190.119 131.572) (end 190.119 125.476) (width 0.16) (layer "F.Cu") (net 6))
 (segment (start 186.182 135.509) (end 190.119 131.572) (width 0.16) (layer "F.Cu") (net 6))
 (segment (start 132.2951 118.7839) (end 132.2951 134.7081) (width 0.16) (layer "F.Cu") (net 6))
 (segment (start 132.2951 99.7339) (end 132.2951 117.9441) (width 0.16) (layer "F.Cu") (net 6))
 (segment (start 132.715 99.314) (end 132.2951 99.7339) (width 0.16) (layer "F.Cu") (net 6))
 (segment (start 132.2951 134.7081) (end 133.096 135.509) (width 0.16) (layer "F.Cu") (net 6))
 (segment (start 132.715 118.364) (end 132.2951 118.7839) (width 0.16) (layer "F.Cu") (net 6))
 (segment (start 189.738 125.222) (end 194.818 120.142) (width 0.16) (layer "F.Cu") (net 2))
 (segment (start 151.3451 99.7339) (end 151.3451 117.9441) (width 0.16) (layer "F.Cu") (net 2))
 (segment (start 151.765 99.314) (end 151.3451 99.7339) (width 0.16) (layer "F.Cu") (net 2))
 (segment (start 186.182 134.874) (end 189.738 131.318) (width 0.16) (layer "F.Cu") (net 2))
 (segment (start 151.257 118.872) (end 151.257 133.731) (width 0.16) (layer "F.Cu") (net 2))
 (segment (start 152.4 134.874) (end 186.182 134.874) (width 0.16) (layer "F.Cu") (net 2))
 (segment (start 151.765 118.364) (end 151.257 118.872) (width 0.16) (layer "F.Cu") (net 2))
 (segment (start 189.738 131.318) (end 189.738 125.222) (width 0.16) (layer "F.Cu") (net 2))
 (segment (start 151.257 133.731) (end 152.4 134.874) (width 0.16) (layer "F.Cu") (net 2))
 (segment (start 194.818 120.142) (end 195.326 120.142) (width 0.16) (layer "F.Cu") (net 2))
 (segment (start 151.3451 117.9441) (end 151.765 118.364) (width 0.16) (layer "F.Cu") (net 2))
 (segment (start 187.96 114.046) (end 192.024 109.982) (width 0.16) (layer "F.Cu") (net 4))
 (segment (start 170.3951 99.7339) (end 170.3951 117.9441) (width 0.16) (layer "F.Cu") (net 4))
 (segment (start 173.482 114.046) (end 187.96 114.046) (width 0.16) (layer "F.Cu") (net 4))
 (segment (start 170.815 118.364) (end 171.831 117.348) (width 0.16) (layer "F.Cu") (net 4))
 (segment (start 170.815 99.314) (end 170.3951 99.7339) (width 0.16) (layer "F.Cu") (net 4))
 (segment (start 170.3951 117.9441) (end 170.815 118.364) (width 0.16) (layer "F.Cu") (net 4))
 (segment (start 171.831 115.697) (end 173.482 114.046) (width 0.16) (layer "F.Cu") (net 4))
 (segment (start 192.024 109.982) (end 195.326 109.982) (width 0.16) (layer "F.Cu") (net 4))
 (segment (start 170.815 118.364) (end 170.307 118.872) (width 0.16) (layer "F.Cu") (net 4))
 (segment (start 171.831 117.348) (end 171.831 115.697) (width 0.16) (layer "F.Cu") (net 4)))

